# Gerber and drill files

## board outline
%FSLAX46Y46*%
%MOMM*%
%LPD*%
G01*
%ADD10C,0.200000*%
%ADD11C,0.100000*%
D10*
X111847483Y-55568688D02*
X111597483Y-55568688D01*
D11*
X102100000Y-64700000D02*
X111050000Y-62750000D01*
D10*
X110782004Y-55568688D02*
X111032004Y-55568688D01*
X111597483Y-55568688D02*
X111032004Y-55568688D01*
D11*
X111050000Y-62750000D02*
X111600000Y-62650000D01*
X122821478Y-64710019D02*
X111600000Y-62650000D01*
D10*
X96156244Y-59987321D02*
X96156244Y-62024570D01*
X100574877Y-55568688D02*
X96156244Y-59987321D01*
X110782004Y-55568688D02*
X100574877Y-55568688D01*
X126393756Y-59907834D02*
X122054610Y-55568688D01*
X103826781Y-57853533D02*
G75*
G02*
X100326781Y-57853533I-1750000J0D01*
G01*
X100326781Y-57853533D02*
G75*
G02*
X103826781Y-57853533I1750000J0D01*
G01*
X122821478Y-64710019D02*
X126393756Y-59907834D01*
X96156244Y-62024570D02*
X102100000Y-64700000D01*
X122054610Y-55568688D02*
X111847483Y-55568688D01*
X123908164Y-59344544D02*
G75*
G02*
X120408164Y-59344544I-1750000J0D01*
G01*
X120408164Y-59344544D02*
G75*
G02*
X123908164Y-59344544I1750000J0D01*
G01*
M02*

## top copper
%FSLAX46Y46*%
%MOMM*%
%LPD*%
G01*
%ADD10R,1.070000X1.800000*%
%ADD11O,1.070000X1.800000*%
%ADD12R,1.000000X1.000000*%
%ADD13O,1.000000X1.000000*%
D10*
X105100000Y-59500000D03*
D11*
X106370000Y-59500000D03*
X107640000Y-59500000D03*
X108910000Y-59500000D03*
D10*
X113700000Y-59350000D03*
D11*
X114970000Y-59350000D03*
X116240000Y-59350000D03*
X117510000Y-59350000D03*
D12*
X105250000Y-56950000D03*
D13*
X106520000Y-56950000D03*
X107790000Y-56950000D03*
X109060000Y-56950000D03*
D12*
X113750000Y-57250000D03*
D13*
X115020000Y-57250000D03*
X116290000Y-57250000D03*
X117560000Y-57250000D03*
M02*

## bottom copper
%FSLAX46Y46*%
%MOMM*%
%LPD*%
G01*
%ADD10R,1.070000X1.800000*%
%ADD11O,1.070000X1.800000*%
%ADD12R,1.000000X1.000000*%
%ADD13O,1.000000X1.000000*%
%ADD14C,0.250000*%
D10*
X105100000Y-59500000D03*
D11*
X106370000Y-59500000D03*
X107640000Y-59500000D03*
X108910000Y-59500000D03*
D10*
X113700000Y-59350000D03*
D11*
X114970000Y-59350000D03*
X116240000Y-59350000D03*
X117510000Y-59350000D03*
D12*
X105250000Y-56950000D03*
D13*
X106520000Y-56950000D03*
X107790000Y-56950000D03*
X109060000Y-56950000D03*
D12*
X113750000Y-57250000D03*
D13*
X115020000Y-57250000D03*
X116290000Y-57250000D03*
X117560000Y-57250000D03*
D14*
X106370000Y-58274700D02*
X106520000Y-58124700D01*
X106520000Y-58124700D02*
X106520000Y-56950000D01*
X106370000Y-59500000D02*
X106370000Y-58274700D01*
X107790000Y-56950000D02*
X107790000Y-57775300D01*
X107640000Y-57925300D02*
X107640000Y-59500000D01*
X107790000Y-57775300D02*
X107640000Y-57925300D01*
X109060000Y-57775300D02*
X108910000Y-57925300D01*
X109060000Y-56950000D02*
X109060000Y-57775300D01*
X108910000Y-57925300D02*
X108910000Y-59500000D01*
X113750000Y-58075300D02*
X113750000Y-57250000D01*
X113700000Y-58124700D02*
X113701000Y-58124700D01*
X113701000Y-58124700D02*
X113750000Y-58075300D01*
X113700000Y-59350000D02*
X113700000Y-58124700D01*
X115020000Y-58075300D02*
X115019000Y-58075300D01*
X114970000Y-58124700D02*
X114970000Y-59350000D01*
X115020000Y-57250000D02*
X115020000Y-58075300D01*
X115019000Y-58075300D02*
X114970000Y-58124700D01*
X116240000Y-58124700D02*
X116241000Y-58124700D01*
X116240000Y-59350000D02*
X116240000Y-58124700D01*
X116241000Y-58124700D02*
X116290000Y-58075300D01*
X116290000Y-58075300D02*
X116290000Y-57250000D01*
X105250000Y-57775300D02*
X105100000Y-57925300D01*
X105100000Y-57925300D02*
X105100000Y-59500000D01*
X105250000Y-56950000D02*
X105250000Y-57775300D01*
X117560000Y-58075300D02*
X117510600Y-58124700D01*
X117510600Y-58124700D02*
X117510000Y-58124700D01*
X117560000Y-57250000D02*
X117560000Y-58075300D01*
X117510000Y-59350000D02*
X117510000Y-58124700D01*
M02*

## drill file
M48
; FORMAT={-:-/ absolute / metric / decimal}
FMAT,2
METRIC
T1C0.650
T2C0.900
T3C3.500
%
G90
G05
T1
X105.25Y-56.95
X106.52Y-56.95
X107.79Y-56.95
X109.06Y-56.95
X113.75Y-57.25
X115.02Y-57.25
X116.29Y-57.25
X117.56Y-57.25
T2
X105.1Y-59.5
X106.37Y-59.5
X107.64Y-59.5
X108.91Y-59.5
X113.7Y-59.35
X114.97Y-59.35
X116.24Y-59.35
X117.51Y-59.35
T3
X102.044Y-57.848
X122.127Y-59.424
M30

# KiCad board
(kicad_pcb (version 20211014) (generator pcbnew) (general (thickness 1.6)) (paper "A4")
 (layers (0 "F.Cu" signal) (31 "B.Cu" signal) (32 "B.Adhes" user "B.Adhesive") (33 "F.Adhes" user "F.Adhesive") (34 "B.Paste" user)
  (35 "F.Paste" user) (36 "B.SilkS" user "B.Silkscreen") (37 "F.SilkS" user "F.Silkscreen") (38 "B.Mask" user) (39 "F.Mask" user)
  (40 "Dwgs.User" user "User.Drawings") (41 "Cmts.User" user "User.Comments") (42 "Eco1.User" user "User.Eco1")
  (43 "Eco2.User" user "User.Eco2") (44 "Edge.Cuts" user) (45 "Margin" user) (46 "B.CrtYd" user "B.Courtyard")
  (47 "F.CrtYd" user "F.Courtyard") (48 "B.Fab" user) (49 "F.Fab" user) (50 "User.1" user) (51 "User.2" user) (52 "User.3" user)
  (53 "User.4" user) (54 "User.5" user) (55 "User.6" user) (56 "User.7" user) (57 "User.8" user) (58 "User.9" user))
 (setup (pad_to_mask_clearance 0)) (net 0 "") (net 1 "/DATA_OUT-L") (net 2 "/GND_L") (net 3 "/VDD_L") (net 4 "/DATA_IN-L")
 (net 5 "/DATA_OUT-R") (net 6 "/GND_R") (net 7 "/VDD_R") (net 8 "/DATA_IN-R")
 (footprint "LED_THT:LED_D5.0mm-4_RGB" (layer "F.Cu") (at 105.1 59.5)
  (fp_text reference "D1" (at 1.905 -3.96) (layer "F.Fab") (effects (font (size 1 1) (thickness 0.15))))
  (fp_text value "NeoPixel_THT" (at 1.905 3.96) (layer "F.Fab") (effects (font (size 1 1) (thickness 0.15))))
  (pad "1" thru_hole rect (at 0 0) (size 1.07 1.8) (drill 0.9) (layers *.Cu *.Mask) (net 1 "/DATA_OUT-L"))
  (pad "2" thru_hole oval (at 1.27 0) (size 1.07 1.8) (drill 0.9) (layers *.Cu *.Mask) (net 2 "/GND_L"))
  (pad "3" thru_hole oval (at 2.54 0) (size 1.07 1.8) (drill 0.9) (layers *.Cu *.Mask) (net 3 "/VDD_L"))
  (pad "4" thru_hole oval (at 3.81 0) (size 1.07 1.8) (drill 0.9) (layers *.Cu *.Mask) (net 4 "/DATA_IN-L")))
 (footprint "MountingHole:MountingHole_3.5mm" (layer "F.Cu") (at 102.044164 57.847931)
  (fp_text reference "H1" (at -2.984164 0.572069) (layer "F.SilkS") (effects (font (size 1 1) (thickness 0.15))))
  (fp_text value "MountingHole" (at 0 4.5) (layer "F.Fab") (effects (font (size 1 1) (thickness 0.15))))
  (pad "" np_thru_hole circle (at 0 0) (size 3.5 3.5) (drill 3.5) (layers *.Cu *.Mask)))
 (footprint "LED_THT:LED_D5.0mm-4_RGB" (layer "F.Cu") (at 113.7 59.35)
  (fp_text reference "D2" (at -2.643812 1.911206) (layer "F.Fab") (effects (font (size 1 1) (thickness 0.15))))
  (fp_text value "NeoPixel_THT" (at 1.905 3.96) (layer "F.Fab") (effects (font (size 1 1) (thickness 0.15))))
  (pad "1" thru_hole rect (at 0 0) (size 1.07 1.8) (drill 0.9) (layers *.Cu *.Mask) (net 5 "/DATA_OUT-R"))
  (pad "2" thru_hole oval (at 1.27 0) (size 1.07 1.8) (drill 0.9) (layers *.Cu *.Mask) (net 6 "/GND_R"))
  (pad "3" thru_hole oval (at 2.54 0) (size 1.07 1.8) (drill 0.9) (layers *.Cu *.Mask) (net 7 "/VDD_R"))
  (pad "4" thru_hole oval (at 3.81 0) (size 1.07 1.8) (drill 0.9) (layers *.Cu *.Mask) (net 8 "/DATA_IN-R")))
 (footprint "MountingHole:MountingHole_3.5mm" (layer "F.Cu") (at 122.12686 59.423927)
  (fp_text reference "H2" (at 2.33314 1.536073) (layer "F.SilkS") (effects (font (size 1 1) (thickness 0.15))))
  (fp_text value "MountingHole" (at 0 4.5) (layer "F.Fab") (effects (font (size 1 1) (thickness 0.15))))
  (pad "" np_thru_hole circle (at 0 0) (size 3.5 3.5) (drill 3.5) (layers *.Cu *.Mask)))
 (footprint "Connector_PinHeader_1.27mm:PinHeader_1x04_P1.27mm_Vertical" (layer "B.Cu") (at 105.25 56.95 -90)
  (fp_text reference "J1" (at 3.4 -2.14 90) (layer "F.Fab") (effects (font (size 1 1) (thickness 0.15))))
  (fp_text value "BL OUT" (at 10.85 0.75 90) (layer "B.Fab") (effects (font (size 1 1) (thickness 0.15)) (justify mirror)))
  (pad "1" thru_hole rect (at 0 0 270) (size 1 1) (drill 0.65) (layers *.Cu *.Mask) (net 1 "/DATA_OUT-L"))
  (pad "2" thru_hole oval (at 0 -1.27 270) (size 1 1) (drill 0.65) (layers *.Cu *.Mask) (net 2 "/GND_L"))
  (pad "3" thru_hole oval (at 0 -2.54 270) (size 1 1) (drill 0.65) (layers *.Cu *.Mask) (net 3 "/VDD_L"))
  (pad "4" thru_hole oval (at 0 -3.81 270) (size 1 1) (drill 0.65) (layers *.Cu *.Mask) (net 4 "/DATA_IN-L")))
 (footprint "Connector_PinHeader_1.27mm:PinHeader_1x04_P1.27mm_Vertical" (layer "B.Cu") (at 113.75 57.25 -90)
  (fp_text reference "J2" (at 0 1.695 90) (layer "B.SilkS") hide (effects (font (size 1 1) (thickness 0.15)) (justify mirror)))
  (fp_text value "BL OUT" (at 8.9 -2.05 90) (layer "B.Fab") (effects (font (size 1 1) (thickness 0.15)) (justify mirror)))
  (pad "1" thru_hole rect (at 0 0 270) (size 1 1) (drill 0.65) (layers *.Cu *.Mask) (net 5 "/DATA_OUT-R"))
  (pad "2" thru_hole oval (at 0 -1.27 270) (size 1 1) (drill 0.65) (layers *.Cu *.Mask) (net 6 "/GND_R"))
  (pad "3" thru_hole oval (at 0 -2.54 270) (size 1 1) (drill 0.65) (layers *.Cu *.Mask) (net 7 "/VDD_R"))
  (pad "4" thru_hole oval (at 0 -3.81 270) (size 1 1) (drill 0.65) (layers *.Cu *.Mask) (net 8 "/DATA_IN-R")))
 (gr_line (start 111.847483 55.568688) (end 111.597483 55.568688) (layer "Edge.Cuts") (width 0.2))
 (gr_line (start 102.1 64.7) (end 111.05 62.75) (layer "Edge.Cuts") (width 0.1))
 (gr_line (start 110.782004 55.568688) (end 111.032004 55.568688) (layer "Edge.Cuts") (width 0.2))
 (gr_line (start 111.597483 55.568688) (end 111.032004 55.568688) (layer "Edge.Cuts") (width 0.2))
 (gr_line (start 111.05 62.75) (end 111.6 62.65) (layer "Edge.Cuts") (width 0.1))
 (gr_line (start 122.821478 64.710019) (end 111.6 62.65) (layer "Edge.Cuts") (width 0.1))
 (gr_line (start 96.156244 59.987321) (end 96.156244 62.02457) (layer "Edge.Cuts") (width 0.2))
 (gr_line (start 100.574877 55.568688) (end 96.156244 59.987321) (layer "Edge.Cuts") (width 0.2))
 (gr_line (start 110.782004 55.568688) (end 100.574877 55.568688) (layer "Edge.Cuts") (width 0.2))
 (gr_line (start 126.393756 59.907834) (end 122.05461 55.568688) (layer "Edge.Cuts") (width 0.2))
 (gr_circle (center 102.076781 57.853533) (end 103.826781 57.853533) (layer "Edge.Cuts") (width 0.2) (fill none))
 (gr_line (start 122.821478 64.710019) (end 126.393756 59.907834) (layer "Edge.Cuts") (width 0.2))
 (gr_line (start 96.156244 62.02457) (end 102.1 64.7) (layer "Edge.Cuts") (width 0.2))
 (gr_line (start 122.05461 55.568688) (end 111.847483 55.568688) (layer "Edge.Cuts") (width 0.2))
 (gr_circle (center 122.158164 59.344544) (end 123.908164 59.344544) (layer "Edge.Cuts") (width 0.2) (fill none))
 (segment (start 106.37 58.2747) (end 106.52 58.1247) (width 0.25) (layer "B.Cu") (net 2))
 (segment (start 106.52 58.1247) (end 106.52 56.95) (width 0.25) (layer "B.Cu") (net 2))
 (segment (start 106.37 59.5) (end 106.37 58.2747) (width 0.25) (layer "B.Cu") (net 2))
 (segment (start 107.79 56.95) (end 107.79 57.7753) (width 0.25) (layer "B.Cu") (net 3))
 (segment (start 107.64 57.9253) (end 107.64 59.5) (width 0.25) (layer "B.Cu") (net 3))
 (segment (start 107.79 57.7753) (end 107.64 57.9253) (width 0.25) (layer "B.Cu") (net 3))
 (segment (start 109.06 57.7753) (end 108.91 57.9253) (width 0.25) (layer "B.Cu") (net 4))
 (segment (start 109.06 56.95) (end 109.06 57.7753) (width 0.25) (layer "B.Cu") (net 4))
 (segment (start 108.91 57.9253) (end 108.91 59.5) (width 0.25) (layer "B.Cu") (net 4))
 (segment (start 113.75 58.0753) (end 113.75 57.25) (width 0.25) (layer "B.Cu") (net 5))
 (segment (start 113.7 58.1247) (end 113.701 58.1247) (width 0.25) (layer "B.Cu") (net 5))
 (segment (start 113.701 58.1247) (end 113.75 58.0753) (width 0.25) (layer "B.Cu") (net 5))
 (segment (start 113.7 59.35) (end 113.7 58.1247) (width 0.25) (layer "B.Cu") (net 5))
 (segment (start 115.02 58.0753) (end 115.019 58.0753) (width 0.25) (layer "B.Cu") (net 6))
 (segment (start 114.97 58.1247) (end 114.97 59.35) (width 0.25) (layer "B.Cu") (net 6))
 (segment (start 115.02 57.25) (end 115.02 58.0753) (width 0.25) (layer "B.Cu") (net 6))
 (segment (start 115.019 58.0753) (end 114.97 58.1247) (width 0.25) (layer "B.Cu") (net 6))
 (segment (start 116.24 58.1247) (end 116.241 58.1247) (width 0.25) (layer "B.Cu") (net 7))
 (segment (start 116.24 59.35) (end 116.24 58.1247) (width 0.25) (layer "B.Cu") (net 7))
 (segment (start 116.241 58.1247) (end 116.29 58.0753) (width 0.25) (layer "B.Cu") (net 7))
 (segment (start 116.29 58.0753) (end 116.29 57.25) (width 0.25) (layer "B.Cu") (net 7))
 (segment (start 105.25 57.7753) (end 105.1 57.9253) (width 0.25) (layer "B.Cu") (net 1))
 (segment (start 105.1 57.9253) (end 105.1 59.5) (width 0.25) (layer "B.Cu") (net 1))
 (segment (start 105.25 56.95) (end 105.25 57.7753) (width 0.25) (layer "B.Cu") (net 1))
 (segment (start 117.56 58.0753) (end 117.5106 58.1247) (width 0.25) (layer "B.Cu") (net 8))
 (segment (start 117.5106 58.1247) (end 117.51 58.1247) (width 0.25) (layer "B.Cu") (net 8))
 (segment (start 117.56 57.25) (end 117.56 58.0753) (width 0.25) (layer "B.Cu") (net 8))
 (segment (start 117.51 59.35) (end 117.51 58.1247) (width 0.25) (layer "B.Cu") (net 8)))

